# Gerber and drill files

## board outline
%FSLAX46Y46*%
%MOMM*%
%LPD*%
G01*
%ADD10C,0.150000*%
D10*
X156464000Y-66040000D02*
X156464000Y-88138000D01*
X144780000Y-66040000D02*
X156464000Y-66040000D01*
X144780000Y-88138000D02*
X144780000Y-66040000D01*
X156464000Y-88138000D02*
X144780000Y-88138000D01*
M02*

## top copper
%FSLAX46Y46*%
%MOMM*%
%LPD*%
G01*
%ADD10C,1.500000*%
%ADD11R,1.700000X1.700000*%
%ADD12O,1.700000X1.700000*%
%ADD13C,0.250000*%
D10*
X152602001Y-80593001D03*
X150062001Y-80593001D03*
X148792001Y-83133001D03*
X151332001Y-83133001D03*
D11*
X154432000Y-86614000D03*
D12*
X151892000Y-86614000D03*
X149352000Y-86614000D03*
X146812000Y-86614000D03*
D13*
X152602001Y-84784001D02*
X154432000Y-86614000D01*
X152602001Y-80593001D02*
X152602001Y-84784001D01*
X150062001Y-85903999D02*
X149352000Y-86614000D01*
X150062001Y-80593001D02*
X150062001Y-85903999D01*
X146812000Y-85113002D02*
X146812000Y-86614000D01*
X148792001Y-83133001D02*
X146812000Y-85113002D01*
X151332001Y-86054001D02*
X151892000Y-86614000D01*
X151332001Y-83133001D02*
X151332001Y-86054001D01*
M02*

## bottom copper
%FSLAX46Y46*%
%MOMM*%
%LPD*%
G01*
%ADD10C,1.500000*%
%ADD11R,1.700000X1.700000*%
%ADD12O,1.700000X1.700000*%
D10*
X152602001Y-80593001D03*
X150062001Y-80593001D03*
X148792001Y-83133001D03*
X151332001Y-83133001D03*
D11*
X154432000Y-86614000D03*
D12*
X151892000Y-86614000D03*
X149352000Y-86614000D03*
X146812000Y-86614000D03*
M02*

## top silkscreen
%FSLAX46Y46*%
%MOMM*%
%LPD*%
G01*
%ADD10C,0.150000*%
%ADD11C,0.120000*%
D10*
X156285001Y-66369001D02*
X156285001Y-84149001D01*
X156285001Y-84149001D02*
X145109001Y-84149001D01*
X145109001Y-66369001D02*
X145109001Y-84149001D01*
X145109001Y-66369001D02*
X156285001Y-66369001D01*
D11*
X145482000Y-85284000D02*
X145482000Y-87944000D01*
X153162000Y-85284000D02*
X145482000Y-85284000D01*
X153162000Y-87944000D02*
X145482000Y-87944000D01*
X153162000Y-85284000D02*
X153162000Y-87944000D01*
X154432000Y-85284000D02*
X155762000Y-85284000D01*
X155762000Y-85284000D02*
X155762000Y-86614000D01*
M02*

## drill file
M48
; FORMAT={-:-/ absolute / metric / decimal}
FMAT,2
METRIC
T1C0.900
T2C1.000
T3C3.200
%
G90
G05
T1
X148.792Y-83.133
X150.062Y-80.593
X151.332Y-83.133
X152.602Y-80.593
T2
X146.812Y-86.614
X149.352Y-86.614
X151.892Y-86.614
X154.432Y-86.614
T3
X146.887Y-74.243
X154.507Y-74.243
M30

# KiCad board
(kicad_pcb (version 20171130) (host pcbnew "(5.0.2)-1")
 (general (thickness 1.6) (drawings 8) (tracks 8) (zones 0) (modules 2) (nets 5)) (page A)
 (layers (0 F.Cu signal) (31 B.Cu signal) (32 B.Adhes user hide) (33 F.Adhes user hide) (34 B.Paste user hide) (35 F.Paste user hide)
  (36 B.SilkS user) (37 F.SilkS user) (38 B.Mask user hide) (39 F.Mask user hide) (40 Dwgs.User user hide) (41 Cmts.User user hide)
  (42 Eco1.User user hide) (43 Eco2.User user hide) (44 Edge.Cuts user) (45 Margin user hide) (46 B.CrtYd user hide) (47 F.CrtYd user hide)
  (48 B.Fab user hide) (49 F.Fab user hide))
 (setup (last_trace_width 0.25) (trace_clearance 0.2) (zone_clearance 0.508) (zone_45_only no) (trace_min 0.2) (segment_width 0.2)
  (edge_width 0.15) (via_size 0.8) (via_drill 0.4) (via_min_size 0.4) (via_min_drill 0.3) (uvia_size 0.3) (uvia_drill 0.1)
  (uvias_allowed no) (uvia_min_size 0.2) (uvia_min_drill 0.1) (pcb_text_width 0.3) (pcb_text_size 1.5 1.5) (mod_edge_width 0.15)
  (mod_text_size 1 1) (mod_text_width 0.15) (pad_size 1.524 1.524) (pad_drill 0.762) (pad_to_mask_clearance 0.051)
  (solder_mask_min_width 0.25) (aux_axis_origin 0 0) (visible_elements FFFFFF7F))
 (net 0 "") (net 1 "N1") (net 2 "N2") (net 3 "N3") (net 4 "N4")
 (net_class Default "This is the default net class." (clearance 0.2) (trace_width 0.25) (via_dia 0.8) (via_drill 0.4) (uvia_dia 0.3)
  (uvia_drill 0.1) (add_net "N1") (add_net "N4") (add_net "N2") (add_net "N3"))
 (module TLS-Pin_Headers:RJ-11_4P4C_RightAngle (layer F.Cu) (at 150.697001 80.593001 180)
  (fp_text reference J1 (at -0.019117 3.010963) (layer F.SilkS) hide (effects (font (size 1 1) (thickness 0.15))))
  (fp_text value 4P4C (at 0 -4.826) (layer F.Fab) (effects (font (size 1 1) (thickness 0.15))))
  (fp_line (start -5.588 14.224) (end -5.588 -3.556) (layer F.SilkS) (width 0.15))
  (fp_line (start -5.588 -3.556) (end 5.588 -3.556) (layer F.SilkS) (width 0.15))
  (fp_line (start 5.588 14.224) (end 5.588 -3.556) (layer F.SilkS) (width 0.15))
  (fp_line (start 5.588 14.224) (end -5.588 14.224) (layer F.SilkS) (width 0.15))
  (pad "" np_thru_hole circle (at -3.81 6.35) (size 3.2 3.2) (drill 3.2) (layers *.Cu *.Mask))
  (pad "" np_thru_hole circle (at 3.81 6.35) (size 3.2 3.2) (drill 3.2) (layers *.Cu *.Mask))
  (pad 1 thru_hole circle (at -1.905 0) (size 1.5 1.5) (drill 0.9) (layers *.Cu *.Mask) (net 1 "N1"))
  (pad 3 thru_hole circle (at 0.635 0) (size 1.5 1.5) (drill 0.9) (layers *.Cu *.Mask) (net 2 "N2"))
  (pad 4 thru_hole circle (at 1.905 -2.54) (size 1.5 1.5) (drill 0.9) (layers *.Cu *.Mask) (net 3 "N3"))
  (pad 2 thru_hole circle (at -0.635 -2.54) (size 1.5 1.5) (drill 0.9) (layers *.Cu *.Mask) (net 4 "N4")))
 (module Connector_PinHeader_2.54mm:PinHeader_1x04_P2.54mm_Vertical (layer F.Cu) (at 154.432 86.614 270)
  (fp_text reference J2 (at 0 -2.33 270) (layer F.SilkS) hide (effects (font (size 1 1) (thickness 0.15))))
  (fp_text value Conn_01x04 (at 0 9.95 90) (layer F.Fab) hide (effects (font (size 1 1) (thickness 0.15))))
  (fp_line (start -1.33 8.95) (end 1.33 8.95) (layer F.SilkS) (width 0.12))
  (fp_line (start -1.33 1.27) (end -1.33 8.95) (layer F.SilkS) (width 0.12))
  (fp_line (start 1.33 1.27) (end 1.33 8.95) (layer F.SilkS) (width 0.12))
  (fp_line (start -1.33 1.27) (end 1.33 1.27) (layer F.SilkS) (width 0.12))
  (fp_line (start -1.33 0) (end -1.33 -1.33) (layer F.SilkS) (width 0.12))
  (fp_line (start -1.33 -1.33) (end 0 -1.33) (layer F.SilkS) (width 0.12))
  (pad 1 thru_hole rect (at 0 0 270) (size 1.7 1.7) (drill 1) (layers *.Cu *.Mask) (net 1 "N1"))
  (pad 2 thru_hole oval (at 0 2.54 270) (size 1.7 1.7) (drill 1) (layers *.Cu *.Mask) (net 4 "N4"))
  (pad 3 thru_hole oval (at 0 5.08 270) (size 1.7 1.7) (drill 1) (layers *.Cu *.Mask) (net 2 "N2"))
  (pad 4 thru_hole oval (at 0 7.62 270) (size 1.7 1.7) (drill 1) (layers *.Cu *.Mask) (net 3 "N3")))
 (gr_line (start 156.464 66.04) (end 156.464 88.138) (layer Edge.Cuts) (width 0.15))
 (gr_line (start 144.78 66.04) (end 156.464 66.04) (layer Edge.Cuts) (width 0.15))
 (gr_line (start 144.78 88.138) (end 144.78 66.04) (layer Edge.Cuts) (width 0.15))
 (gr_line (start 156.464 88.138) (end 144.78 88.138) (layer Edge.Cuts) (width 0.15))
 (segment (start 152.602001 84.784001) (end 154.432 86.614) (width 0.25) (layer F.Cu) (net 1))
 (segment (start 152.602001 80.593001) (end 152.602001 84.784001) (width 0.25) (layer F.Cu) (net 1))
 (segment (start 150.062001 85.903999) (end 149.352 86.614) (width 0.25) (layer F.Cu) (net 2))
 (segment (start 150.062001 80.593001) (end 150.062001 85.903999) (width 0.25) (layer F.Cu) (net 2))
 (segment (start 146.812 85.113002) (end 146.812 86.614) (width 0.25) (layer F.Cu) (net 3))
 (segment (start 148.792001 83.133001) (end 146.812 85.113002) (width 0.25) (layer F.Cu) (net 3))
 (segment (start 151.332001 86.054001) (end 151.892 86.614) (width 0.25) (layer F.Cu) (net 4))
 (segment (start 151.332001 83.133001) (end 151.332001 86.054001) (width 0.25) (layer F.Cu) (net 4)))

